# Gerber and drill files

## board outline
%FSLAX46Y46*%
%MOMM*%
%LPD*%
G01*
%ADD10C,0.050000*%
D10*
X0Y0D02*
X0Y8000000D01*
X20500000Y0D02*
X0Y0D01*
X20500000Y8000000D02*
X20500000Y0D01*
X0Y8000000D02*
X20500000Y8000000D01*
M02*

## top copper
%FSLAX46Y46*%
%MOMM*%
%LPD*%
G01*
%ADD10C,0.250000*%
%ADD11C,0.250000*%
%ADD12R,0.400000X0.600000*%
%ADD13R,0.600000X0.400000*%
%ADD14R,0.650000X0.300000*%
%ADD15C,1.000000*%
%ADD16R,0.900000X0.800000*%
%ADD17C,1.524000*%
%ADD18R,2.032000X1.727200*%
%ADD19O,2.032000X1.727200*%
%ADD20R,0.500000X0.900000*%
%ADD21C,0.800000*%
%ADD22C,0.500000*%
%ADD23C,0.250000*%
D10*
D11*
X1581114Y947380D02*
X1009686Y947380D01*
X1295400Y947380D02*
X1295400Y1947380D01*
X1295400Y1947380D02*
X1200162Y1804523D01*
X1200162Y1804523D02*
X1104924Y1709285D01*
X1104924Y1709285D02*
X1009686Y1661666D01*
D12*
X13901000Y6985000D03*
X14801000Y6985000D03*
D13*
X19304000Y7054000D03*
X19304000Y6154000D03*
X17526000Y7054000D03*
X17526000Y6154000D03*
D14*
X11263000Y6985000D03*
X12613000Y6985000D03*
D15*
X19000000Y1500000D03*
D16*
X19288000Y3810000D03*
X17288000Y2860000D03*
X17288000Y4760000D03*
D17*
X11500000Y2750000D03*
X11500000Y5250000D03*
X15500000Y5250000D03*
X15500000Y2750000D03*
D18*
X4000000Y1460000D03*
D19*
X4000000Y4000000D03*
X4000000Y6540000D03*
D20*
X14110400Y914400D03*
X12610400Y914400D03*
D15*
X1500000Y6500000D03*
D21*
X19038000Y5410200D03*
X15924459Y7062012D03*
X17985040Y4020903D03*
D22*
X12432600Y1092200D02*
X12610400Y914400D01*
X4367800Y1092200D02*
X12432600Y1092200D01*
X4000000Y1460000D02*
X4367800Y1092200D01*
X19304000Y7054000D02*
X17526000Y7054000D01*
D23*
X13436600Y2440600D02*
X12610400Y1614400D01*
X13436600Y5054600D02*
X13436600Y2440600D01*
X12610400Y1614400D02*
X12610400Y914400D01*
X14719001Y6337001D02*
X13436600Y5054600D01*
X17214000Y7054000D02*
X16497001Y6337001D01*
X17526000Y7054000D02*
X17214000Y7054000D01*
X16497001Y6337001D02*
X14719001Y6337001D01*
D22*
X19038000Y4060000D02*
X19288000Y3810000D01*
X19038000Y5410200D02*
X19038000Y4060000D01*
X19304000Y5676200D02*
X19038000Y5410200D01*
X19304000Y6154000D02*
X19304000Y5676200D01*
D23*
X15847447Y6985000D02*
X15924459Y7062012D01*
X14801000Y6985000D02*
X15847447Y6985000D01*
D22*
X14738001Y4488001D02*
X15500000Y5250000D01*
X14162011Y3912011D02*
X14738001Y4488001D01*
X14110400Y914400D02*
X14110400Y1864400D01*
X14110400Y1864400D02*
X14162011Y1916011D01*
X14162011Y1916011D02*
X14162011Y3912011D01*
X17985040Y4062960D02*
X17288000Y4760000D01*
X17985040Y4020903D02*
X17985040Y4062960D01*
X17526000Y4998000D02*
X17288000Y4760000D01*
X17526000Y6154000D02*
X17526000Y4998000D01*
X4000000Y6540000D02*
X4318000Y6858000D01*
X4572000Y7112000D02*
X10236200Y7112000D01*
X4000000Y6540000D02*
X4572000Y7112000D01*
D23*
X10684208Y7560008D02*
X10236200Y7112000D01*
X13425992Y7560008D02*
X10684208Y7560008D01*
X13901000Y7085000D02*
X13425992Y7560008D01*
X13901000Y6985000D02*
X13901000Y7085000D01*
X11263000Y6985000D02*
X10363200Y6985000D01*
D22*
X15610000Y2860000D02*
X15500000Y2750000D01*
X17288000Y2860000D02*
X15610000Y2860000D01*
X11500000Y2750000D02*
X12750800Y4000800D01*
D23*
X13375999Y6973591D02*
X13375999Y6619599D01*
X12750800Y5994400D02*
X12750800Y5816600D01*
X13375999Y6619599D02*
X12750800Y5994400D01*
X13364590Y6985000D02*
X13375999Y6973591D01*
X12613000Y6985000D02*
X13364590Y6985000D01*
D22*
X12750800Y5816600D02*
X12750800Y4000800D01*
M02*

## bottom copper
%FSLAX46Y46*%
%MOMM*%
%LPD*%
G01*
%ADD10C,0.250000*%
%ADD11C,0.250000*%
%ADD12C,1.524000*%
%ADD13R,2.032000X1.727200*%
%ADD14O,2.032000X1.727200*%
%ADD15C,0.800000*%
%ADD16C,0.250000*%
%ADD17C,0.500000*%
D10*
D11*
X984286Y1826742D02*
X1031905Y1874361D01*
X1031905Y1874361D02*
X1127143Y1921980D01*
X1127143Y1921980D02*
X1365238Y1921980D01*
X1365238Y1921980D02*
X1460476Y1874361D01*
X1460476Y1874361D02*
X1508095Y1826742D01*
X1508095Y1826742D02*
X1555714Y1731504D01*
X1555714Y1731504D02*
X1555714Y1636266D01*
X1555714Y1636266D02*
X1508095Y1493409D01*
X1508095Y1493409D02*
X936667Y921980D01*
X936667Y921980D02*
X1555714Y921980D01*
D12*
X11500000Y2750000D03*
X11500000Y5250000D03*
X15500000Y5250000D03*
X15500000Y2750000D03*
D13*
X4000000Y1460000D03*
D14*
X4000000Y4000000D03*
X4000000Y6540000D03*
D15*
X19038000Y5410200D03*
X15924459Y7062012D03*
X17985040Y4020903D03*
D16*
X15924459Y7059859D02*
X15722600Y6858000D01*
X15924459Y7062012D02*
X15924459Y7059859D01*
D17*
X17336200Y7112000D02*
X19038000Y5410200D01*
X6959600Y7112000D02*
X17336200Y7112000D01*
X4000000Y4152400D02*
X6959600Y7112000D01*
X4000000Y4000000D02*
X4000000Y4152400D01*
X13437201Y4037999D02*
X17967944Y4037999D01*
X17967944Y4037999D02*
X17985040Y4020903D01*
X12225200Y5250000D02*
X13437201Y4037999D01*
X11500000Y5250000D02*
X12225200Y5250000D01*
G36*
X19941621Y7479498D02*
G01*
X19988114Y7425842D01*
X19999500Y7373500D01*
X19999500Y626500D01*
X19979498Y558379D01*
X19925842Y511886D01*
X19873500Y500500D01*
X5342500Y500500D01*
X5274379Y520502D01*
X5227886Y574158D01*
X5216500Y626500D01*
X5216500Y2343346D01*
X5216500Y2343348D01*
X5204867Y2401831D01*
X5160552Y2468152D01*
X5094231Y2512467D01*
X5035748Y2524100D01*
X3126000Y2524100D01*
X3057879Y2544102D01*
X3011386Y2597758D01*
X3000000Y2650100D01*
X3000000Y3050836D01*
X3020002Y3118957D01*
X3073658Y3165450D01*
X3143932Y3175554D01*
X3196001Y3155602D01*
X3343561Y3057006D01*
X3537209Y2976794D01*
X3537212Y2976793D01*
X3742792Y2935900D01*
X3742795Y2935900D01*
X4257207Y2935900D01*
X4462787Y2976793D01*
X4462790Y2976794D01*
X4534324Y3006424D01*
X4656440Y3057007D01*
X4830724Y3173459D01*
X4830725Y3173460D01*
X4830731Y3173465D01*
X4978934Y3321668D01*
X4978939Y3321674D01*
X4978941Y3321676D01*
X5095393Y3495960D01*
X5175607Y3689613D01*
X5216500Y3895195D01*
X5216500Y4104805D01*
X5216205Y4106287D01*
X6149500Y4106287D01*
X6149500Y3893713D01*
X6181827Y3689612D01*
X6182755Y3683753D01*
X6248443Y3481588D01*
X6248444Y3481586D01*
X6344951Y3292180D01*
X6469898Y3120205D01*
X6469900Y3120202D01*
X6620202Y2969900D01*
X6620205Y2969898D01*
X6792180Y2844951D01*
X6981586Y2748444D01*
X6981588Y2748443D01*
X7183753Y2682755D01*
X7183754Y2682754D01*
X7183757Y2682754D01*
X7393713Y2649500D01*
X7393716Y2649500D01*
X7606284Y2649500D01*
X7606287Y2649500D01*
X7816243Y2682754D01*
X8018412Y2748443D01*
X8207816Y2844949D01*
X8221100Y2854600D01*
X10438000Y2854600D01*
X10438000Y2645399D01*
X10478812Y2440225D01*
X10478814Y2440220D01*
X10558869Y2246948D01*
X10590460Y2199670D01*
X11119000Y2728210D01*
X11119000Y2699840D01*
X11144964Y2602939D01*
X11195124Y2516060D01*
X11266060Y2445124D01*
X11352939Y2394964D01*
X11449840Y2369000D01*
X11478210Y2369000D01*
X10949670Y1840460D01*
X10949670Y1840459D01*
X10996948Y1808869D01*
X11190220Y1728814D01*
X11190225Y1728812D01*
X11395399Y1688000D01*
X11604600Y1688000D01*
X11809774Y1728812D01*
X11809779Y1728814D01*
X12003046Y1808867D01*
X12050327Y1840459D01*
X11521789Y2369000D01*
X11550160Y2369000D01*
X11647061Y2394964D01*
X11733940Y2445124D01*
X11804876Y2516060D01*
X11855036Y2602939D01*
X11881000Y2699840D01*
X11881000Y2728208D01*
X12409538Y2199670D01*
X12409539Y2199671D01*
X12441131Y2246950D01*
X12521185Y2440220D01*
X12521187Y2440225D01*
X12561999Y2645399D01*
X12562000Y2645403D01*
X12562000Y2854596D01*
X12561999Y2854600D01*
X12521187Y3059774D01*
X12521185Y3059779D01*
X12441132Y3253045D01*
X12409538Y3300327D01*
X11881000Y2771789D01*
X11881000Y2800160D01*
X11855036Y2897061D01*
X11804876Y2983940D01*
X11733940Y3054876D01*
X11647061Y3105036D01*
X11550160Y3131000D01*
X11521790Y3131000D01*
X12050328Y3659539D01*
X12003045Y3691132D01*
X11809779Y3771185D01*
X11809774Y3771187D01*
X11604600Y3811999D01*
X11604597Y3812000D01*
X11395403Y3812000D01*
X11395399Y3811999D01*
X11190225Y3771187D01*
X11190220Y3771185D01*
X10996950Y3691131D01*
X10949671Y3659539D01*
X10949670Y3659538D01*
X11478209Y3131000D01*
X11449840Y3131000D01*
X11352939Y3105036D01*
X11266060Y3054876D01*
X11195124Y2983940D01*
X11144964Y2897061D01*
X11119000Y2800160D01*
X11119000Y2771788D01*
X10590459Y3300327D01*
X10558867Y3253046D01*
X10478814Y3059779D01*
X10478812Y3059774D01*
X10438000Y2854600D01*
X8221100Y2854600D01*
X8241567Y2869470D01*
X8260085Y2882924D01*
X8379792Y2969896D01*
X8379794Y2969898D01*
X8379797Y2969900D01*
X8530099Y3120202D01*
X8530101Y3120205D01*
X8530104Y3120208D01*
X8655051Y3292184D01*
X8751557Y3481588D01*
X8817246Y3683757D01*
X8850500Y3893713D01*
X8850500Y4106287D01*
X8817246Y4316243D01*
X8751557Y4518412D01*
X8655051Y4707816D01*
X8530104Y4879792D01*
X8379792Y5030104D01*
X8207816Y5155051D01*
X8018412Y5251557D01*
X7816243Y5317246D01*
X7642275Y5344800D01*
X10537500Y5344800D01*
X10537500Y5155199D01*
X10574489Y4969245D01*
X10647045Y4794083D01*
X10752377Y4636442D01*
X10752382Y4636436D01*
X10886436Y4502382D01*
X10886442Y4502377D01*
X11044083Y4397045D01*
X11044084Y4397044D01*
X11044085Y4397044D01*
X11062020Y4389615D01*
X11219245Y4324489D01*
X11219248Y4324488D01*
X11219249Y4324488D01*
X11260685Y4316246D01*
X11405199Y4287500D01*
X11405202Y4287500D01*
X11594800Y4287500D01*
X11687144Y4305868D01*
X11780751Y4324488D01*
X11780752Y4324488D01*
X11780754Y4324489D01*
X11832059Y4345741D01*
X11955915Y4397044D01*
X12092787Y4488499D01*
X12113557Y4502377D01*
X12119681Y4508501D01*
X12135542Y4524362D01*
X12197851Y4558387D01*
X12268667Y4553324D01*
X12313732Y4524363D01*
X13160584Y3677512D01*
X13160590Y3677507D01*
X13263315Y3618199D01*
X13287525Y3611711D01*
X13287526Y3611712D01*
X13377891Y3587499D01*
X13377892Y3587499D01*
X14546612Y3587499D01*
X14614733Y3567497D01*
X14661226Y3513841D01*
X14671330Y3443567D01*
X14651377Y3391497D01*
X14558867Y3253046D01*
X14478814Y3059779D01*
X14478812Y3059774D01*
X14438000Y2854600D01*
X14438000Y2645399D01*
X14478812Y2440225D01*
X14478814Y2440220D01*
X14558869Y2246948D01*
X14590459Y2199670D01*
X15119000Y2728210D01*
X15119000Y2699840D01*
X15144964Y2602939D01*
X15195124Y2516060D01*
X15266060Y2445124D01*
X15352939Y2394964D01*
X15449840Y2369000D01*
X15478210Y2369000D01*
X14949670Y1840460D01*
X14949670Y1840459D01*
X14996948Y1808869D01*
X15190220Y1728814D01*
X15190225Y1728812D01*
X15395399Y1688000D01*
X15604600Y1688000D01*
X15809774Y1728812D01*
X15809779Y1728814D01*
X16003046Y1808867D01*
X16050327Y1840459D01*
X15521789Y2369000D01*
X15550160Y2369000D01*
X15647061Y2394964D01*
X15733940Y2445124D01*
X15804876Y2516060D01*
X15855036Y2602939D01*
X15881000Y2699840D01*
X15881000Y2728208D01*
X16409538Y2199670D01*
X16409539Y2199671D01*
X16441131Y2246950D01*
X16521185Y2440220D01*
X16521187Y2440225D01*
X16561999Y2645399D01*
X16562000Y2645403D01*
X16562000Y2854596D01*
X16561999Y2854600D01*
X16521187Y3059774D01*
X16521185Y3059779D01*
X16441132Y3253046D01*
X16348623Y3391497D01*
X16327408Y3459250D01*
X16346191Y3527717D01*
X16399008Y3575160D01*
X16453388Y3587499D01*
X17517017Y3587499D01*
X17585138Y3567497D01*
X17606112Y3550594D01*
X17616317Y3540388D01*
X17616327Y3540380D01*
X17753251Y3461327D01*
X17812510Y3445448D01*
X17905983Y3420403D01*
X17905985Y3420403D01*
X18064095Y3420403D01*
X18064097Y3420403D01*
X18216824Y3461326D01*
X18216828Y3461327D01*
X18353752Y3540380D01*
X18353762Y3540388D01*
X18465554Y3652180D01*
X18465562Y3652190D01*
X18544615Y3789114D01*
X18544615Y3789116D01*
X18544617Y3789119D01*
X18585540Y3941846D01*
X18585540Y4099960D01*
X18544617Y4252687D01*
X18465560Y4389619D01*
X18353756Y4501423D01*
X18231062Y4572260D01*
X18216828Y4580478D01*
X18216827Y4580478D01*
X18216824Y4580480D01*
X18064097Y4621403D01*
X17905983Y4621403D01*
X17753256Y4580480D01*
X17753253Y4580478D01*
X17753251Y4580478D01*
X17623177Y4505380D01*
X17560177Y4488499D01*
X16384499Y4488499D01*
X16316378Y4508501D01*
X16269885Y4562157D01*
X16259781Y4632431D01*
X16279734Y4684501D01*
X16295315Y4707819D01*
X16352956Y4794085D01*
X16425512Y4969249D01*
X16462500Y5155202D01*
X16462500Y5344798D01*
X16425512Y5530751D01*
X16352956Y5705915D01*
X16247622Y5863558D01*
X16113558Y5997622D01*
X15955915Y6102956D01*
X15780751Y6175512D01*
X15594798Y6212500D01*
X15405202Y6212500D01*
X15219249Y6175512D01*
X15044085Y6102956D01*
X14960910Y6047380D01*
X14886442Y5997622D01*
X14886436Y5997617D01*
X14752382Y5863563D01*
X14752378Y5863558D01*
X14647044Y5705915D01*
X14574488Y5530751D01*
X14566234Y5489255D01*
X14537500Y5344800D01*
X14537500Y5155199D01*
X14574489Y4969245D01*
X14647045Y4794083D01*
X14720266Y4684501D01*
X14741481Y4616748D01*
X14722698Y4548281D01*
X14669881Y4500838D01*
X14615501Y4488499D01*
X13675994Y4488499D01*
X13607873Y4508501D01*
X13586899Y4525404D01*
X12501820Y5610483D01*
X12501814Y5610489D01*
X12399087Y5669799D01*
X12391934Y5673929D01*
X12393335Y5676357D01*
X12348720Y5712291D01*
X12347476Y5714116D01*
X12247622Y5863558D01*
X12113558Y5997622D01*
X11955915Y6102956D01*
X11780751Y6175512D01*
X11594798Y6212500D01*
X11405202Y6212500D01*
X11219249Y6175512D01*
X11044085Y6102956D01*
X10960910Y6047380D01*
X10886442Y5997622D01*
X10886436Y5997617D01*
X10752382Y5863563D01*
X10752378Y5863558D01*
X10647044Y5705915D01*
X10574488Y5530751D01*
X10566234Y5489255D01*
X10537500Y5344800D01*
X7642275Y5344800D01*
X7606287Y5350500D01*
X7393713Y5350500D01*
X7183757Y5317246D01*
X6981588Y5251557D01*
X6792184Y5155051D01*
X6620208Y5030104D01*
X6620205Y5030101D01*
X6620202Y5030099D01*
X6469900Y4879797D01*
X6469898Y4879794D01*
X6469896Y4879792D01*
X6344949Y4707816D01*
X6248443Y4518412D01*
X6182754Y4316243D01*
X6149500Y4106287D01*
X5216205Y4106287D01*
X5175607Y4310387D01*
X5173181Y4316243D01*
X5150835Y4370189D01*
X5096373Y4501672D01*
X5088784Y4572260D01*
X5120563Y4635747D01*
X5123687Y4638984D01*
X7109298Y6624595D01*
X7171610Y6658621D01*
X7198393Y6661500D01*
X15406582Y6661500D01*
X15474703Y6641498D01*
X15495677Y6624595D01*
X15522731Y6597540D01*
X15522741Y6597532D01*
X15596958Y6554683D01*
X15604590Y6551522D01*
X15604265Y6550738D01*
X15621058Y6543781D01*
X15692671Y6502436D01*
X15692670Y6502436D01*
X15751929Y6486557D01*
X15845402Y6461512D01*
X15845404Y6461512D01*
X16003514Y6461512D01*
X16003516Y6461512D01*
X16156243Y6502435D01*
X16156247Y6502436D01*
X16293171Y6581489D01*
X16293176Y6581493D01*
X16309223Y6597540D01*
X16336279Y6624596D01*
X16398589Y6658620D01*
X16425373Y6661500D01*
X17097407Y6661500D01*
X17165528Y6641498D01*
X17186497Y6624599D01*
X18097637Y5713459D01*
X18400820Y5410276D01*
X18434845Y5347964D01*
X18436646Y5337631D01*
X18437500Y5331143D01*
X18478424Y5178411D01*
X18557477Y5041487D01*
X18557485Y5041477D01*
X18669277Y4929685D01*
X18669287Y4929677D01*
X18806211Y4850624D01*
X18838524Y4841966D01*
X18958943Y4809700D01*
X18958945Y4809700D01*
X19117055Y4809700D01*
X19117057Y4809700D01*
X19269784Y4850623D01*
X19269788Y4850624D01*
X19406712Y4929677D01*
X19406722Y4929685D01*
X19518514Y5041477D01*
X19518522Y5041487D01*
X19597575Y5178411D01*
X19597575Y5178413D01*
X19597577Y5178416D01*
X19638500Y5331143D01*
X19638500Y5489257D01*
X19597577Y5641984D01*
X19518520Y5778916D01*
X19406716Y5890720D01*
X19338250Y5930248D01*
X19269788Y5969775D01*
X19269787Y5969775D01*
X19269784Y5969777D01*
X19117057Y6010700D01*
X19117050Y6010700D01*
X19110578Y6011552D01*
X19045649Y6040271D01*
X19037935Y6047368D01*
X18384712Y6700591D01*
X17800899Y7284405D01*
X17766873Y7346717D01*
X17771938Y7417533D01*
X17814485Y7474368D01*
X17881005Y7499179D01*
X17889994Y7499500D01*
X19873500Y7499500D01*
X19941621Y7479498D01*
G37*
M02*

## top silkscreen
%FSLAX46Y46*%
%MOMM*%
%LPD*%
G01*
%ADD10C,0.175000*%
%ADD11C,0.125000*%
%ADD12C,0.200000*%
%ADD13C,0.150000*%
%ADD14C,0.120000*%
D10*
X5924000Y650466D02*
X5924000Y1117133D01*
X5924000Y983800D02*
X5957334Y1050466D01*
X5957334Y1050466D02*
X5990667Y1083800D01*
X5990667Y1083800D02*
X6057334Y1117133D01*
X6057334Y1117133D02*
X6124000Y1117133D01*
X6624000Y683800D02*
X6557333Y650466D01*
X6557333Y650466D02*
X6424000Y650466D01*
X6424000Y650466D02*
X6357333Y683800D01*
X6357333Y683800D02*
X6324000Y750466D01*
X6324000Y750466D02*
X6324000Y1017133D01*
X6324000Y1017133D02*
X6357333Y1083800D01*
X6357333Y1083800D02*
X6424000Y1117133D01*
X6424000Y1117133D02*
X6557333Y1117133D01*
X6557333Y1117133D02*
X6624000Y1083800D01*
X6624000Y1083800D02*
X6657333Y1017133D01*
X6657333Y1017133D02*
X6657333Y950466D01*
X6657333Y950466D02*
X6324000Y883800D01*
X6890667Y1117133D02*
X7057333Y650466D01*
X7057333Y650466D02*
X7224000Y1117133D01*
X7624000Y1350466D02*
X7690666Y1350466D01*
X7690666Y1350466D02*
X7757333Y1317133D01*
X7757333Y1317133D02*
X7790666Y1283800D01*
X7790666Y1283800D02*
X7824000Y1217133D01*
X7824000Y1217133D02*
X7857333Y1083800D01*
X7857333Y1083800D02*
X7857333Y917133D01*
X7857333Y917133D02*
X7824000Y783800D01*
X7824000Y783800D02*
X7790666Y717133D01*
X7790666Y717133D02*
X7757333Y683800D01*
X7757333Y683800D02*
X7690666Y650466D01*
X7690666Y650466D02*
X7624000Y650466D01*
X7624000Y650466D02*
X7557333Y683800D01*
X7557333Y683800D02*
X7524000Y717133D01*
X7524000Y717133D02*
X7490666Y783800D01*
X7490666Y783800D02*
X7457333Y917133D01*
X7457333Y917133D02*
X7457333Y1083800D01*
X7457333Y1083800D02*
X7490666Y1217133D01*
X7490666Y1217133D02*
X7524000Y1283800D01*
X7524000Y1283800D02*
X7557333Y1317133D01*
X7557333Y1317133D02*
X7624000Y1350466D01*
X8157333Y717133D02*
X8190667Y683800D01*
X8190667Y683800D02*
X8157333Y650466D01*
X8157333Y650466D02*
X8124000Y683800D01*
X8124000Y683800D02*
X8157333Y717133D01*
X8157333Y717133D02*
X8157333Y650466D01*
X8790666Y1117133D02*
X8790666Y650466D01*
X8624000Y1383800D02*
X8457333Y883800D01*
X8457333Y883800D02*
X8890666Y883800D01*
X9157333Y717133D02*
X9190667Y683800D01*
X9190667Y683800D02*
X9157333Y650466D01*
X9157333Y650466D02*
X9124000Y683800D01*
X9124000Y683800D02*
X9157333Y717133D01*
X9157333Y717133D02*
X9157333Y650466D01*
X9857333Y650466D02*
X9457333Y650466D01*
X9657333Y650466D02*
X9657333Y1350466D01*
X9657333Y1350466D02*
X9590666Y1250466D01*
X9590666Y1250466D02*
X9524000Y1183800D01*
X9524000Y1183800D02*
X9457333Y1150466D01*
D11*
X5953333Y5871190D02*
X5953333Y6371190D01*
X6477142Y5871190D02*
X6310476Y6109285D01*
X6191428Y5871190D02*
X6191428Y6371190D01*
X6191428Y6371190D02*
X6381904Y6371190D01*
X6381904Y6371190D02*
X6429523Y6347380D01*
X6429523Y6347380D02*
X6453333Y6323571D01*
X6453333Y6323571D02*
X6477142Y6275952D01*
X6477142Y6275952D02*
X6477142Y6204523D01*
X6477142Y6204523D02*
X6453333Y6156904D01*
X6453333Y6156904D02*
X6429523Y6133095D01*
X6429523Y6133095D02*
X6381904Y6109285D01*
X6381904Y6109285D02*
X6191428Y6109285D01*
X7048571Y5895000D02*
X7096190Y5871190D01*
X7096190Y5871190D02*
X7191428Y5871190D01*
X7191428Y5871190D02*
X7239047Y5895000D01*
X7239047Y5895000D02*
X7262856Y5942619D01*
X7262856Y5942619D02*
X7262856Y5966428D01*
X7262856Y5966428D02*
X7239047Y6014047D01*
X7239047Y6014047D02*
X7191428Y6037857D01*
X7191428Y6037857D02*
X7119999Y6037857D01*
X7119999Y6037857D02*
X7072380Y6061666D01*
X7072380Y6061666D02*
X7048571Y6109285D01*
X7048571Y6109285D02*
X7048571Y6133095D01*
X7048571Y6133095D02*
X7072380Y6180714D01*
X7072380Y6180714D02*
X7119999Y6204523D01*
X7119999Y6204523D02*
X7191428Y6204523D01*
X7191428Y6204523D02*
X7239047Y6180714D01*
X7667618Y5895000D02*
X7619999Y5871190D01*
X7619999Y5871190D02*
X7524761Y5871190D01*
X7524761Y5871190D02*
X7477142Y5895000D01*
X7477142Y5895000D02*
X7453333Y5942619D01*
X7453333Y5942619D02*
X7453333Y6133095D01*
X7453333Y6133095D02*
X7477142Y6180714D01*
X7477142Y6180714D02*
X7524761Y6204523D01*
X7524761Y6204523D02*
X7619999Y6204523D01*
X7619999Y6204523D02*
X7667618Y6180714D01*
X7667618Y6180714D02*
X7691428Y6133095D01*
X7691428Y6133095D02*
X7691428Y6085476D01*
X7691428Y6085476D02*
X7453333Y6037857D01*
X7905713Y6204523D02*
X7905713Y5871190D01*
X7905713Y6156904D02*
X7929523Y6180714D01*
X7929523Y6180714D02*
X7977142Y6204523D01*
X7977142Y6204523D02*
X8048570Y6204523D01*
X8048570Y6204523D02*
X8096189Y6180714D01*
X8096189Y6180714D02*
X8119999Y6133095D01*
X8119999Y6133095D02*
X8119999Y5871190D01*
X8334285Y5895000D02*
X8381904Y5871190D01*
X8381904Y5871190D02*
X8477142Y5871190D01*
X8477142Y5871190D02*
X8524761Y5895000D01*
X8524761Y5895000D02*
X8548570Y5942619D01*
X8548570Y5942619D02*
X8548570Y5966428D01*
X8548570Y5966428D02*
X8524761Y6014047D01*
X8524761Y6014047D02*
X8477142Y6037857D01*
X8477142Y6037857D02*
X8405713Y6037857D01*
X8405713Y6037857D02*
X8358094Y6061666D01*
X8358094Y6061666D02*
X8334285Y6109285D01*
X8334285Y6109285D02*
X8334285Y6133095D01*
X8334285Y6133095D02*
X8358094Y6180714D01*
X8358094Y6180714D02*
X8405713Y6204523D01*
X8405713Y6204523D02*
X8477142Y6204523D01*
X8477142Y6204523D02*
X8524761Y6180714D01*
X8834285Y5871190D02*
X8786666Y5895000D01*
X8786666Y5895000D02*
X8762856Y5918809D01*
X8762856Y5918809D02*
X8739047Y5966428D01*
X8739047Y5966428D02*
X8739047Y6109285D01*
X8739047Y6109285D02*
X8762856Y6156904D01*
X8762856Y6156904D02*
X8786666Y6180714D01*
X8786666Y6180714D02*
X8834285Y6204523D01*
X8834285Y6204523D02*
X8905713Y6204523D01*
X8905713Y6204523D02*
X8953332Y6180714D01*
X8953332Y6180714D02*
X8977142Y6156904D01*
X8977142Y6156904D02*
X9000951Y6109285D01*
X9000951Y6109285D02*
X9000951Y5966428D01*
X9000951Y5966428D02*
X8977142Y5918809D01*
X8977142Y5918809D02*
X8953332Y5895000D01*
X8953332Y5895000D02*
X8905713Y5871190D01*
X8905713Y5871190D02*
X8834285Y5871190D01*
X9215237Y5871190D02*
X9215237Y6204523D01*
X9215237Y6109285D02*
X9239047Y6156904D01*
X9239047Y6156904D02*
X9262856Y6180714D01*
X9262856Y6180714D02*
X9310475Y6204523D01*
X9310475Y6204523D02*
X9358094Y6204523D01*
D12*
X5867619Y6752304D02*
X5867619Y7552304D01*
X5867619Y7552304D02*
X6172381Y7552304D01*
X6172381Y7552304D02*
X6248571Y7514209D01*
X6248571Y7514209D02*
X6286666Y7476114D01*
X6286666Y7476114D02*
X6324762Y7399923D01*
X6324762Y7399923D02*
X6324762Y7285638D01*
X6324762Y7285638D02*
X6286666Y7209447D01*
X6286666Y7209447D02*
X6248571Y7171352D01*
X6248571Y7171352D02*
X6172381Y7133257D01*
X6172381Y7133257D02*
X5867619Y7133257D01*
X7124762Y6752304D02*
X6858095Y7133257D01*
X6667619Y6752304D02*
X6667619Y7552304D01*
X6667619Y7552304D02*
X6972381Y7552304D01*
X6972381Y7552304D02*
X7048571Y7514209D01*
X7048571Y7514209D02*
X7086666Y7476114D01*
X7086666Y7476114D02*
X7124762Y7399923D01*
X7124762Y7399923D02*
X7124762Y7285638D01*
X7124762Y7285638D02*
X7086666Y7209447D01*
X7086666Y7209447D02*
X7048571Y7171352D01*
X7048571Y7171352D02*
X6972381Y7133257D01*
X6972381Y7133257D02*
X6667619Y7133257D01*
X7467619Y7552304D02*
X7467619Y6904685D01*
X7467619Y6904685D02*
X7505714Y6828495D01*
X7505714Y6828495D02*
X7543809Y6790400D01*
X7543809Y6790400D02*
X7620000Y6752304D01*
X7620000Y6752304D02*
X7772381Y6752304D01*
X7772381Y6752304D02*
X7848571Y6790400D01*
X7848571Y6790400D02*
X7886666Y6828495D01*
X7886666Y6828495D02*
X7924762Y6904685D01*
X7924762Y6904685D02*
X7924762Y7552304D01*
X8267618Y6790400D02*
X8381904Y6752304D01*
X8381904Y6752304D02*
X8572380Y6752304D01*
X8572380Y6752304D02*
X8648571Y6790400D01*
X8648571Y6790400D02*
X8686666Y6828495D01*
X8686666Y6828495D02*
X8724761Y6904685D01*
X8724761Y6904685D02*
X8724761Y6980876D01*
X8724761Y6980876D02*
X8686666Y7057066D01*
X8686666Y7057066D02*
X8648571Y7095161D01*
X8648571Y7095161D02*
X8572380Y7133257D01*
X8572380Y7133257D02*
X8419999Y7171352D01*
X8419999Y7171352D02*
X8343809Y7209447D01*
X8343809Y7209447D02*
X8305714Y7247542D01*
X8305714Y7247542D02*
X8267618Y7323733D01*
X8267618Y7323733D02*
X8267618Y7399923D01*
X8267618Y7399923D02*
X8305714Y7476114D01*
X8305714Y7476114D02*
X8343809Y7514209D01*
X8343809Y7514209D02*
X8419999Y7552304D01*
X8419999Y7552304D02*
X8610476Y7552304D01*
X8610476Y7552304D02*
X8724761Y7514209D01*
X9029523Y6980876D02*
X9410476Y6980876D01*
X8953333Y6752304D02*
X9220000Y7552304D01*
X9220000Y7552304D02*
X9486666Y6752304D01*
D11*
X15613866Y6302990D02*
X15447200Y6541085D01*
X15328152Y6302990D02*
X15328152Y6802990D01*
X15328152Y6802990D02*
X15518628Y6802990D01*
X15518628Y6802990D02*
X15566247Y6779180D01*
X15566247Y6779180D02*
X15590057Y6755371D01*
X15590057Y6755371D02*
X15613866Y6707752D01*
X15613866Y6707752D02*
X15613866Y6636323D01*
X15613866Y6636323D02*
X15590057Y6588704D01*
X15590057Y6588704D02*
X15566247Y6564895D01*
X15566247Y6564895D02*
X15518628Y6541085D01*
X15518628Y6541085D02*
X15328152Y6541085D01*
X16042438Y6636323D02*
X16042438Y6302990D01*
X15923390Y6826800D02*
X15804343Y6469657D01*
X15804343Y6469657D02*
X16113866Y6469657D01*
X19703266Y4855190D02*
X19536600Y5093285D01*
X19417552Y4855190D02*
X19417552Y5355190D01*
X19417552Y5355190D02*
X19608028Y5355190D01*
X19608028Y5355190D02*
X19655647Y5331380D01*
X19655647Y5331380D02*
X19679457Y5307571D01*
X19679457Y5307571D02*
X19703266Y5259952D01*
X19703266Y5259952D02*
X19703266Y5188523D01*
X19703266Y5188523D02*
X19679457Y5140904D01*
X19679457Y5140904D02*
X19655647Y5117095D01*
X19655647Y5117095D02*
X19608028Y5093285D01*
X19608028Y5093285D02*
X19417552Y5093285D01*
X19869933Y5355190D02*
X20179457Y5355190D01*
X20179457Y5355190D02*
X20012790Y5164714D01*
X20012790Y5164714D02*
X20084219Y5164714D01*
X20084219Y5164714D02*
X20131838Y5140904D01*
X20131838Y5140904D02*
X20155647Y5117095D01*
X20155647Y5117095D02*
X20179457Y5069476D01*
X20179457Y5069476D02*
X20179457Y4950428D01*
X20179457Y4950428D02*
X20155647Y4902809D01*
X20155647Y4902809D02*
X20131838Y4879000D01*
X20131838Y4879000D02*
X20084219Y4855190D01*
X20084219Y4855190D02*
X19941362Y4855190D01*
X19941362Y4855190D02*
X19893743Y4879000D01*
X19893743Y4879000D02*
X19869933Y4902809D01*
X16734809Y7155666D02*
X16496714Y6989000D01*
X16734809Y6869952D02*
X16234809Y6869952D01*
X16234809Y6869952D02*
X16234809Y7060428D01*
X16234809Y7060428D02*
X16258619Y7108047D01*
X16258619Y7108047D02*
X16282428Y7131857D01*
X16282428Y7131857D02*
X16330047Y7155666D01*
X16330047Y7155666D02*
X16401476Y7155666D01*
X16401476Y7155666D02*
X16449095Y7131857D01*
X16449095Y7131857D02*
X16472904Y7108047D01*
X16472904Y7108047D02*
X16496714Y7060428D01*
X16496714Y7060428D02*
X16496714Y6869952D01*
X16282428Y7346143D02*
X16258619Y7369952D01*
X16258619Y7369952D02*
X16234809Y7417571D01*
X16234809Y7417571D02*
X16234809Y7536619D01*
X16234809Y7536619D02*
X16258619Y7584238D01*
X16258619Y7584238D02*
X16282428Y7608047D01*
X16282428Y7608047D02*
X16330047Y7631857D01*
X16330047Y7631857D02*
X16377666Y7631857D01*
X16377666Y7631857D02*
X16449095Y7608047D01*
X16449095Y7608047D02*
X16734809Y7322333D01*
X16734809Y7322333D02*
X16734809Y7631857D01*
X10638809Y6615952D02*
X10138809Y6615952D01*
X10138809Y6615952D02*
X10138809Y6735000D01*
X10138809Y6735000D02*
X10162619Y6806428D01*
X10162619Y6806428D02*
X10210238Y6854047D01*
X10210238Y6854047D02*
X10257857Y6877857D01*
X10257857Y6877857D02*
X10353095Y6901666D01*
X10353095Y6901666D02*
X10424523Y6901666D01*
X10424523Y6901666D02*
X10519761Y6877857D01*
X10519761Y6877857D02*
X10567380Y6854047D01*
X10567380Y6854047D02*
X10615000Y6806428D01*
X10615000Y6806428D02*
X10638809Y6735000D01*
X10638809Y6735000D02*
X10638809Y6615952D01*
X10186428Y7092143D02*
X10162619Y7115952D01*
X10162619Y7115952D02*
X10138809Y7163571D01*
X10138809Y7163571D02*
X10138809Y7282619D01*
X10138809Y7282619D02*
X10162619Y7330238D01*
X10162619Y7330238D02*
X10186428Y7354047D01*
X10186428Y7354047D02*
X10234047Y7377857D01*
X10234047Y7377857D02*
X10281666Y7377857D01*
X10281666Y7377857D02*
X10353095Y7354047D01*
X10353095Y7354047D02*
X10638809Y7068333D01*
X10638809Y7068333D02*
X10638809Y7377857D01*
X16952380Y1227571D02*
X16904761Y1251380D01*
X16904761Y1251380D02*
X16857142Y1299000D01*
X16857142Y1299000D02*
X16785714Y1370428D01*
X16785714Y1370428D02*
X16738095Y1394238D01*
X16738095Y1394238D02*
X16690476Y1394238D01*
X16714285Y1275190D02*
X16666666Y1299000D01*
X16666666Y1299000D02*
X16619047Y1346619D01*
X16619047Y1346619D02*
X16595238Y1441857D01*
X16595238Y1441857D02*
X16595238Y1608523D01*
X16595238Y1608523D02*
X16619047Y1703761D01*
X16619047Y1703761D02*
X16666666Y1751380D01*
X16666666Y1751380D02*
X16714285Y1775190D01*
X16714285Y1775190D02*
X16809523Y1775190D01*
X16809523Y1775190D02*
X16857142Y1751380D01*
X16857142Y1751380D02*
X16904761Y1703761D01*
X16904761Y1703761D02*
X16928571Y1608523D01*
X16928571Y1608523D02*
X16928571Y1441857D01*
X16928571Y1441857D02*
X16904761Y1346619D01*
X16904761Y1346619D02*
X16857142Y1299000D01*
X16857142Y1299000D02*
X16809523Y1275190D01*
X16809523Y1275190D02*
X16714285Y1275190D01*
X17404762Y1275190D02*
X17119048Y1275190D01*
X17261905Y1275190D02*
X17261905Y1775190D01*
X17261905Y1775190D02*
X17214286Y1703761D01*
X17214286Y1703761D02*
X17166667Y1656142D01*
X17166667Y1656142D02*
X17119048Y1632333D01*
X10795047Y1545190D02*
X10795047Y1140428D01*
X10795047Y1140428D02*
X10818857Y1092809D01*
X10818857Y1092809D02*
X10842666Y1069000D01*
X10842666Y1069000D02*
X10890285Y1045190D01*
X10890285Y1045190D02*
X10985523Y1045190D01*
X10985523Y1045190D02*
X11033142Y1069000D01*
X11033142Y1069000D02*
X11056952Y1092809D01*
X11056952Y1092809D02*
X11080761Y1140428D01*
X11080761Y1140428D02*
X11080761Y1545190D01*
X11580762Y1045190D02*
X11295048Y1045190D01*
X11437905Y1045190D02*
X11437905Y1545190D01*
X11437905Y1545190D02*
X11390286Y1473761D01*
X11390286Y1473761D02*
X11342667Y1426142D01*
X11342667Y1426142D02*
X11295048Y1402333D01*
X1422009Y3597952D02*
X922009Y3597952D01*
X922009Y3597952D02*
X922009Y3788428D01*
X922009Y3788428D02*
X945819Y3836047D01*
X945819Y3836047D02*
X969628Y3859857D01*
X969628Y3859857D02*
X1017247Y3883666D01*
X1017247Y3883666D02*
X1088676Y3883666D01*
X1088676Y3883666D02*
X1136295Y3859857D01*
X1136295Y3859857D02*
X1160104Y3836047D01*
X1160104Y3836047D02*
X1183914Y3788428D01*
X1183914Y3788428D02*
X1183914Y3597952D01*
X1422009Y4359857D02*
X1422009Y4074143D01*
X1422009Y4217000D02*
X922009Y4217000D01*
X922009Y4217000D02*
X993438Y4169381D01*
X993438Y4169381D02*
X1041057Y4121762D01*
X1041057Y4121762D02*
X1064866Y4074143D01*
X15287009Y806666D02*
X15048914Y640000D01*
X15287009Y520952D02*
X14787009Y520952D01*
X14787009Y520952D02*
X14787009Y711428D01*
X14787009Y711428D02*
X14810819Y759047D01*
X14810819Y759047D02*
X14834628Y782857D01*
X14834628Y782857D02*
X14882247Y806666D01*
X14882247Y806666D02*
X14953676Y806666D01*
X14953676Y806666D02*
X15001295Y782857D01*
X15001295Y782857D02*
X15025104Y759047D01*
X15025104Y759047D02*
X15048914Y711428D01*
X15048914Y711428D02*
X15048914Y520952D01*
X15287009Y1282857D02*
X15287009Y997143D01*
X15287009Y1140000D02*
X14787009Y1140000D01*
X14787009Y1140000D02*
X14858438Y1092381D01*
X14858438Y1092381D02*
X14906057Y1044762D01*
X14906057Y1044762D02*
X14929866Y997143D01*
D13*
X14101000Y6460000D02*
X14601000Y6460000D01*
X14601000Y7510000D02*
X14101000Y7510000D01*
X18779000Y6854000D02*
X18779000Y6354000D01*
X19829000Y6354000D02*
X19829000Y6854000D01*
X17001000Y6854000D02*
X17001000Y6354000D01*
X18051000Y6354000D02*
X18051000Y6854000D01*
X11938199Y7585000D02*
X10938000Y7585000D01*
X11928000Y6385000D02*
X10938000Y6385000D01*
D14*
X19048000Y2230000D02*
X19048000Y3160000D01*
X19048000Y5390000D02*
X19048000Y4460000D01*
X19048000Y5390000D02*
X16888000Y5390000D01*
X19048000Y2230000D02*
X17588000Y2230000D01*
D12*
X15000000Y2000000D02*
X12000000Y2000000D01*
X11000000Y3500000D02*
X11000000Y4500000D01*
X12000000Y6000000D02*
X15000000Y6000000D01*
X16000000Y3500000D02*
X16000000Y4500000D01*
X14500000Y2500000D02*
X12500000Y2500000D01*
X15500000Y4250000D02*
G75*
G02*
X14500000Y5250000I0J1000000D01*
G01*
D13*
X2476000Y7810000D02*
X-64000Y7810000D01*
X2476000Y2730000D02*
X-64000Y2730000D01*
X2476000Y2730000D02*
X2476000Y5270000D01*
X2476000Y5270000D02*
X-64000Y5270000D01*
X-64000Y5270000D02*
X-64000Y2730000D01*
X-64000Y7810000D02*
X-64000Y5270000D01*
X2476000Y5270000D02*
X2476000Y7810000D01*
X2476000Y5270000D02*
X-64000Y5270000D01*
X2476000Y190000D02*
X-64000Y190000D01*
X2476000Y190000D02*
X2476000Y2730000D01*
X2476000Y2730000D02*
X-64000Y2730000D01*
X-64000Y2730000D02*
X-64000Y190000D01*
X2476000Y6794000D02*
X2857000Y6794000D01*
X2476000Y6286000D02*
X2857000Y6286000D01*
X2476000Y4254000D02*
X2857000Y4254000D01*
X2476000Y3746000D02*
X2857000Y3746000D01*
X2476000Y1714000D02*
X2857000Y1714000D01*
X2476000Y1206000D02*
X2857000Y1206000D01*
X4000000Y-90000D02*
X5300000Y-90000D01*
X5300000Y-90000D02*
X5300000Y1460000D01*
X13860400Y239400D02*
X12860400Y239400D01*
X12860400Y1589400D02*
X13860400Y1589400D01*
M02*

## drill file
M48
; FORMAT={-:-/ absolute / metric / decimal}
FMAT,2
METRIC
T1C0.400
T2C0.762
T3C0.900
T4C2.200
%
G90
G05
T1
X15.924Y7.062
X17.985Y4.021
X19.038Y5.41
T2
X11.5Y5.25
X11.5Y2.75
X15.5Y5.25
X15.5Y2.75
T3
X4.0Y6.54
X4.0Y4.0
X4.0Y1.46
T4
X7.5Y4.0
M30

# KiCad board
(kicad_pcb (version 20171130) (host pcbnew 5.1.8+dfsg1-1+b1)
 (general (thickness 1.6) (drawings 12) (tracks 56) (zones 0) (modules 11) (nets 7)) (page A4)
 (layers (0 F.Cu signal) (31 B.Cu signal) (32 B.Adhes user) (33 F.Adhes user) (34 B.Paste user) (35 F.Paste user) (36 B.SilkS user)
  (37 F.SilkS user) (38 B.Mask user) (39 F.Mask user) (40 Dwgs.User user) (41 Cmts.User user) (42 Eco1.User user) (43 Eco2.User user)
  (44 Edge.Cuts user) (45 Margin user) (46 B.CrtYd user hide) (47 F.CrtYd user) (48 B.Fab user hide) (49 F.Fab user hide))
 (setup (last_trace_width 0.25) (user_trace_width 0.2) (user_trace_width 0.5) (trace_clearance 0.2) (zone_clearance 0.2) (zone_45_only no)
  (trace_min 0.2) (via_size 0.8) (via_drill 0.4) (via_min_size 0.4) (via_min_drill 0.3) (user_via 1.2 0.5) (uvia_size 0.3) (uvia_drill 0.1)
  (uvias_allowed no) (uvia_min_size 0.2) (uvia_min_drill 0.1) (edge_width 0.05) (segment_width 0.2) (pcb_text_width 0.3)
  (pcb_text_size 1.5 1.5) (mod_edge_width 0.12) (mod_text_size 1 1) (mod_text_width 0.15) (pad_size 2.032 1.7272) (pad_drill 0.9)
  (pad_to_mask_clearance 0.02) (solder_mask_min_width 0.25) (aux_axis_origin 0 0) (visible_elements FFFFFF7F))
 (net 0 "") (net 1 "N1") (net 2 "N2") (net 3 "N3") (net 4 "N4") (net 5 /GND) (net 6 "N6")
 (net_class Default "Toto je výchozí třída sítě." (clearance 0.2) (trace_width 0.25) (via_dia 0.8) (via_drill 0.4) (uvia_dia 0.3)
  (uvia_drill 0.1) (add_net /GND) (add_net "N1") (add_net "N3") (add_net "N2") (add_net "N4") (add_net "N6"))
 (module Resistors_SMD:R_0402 (layer F.Cu) (at 14.351 -6.985)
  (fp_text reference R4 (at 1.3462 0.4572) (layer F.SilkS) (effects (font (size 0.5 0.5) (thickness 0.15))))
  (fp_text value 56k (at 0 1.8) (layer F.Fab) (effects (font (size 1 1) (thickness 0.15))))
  (fp_line (start -0.25 0.525) (end 0.25 0.525) (layer F.SilkS) (width 0.15))
  (fp_line (start 0.25 -0.525) (end -0.25 -0.525) (layer F.SilkS) (width 0.15))
  (pad 1 smd rect (at -0.45 0) (size 0.4 0.6) (layers F.Cu F.Paste F.Mask) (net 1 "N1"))
  (pad 2 smd rect (at 0.45 0) (size 0.4 0.6) (layers F.Cu F.Paste F.Mask) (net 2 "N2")))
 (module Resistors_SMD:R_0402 (layer F.Cu) (at 19.304 -6.604 90)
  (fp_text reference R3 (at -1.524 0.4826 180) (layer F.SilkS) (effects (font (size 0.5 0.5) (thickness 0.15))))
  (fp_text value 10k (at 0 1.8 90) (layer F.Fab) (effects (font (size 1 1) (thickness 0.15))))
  (fp_line (start 0.25 -0.525) (end -0.25 -0.525) (layer F.SilkS) (width 0.15))
  (fp_line (start -0.25 0.525) (end 0.25 0.525) (layer F.SilkS) (width 0.15))
  (pad 2 smd rect (at 0.45 0 90) (size 0.4 0.6) (layers F.Cu F.Paste F.Mask) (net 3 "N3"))
  (pad 1 smd rect (at -0.45 0 90) (size 0.4 0.6) (layers F.Cu F.Paste F.Mask) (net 2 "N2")))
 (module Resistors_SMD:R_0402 (layer F.Cu) (at 17.526 -6.604 270)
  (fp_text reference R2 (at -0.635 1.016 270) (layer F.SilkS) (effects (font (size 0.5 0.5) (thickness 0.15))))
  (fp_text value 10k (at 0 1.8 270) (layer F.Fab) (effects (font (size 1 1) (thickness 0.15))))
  (fp_line (start -0.25 0.525) (end 0.25 0.525) (layer F.SilkS) (width 0.15))
  (fp_line (start 0.25 -0.525) (end -0.25 -0.525) (layer F.SilkS) (width 0.15))
  (pad 1 smd rect (at -0.45 0 270) (size 0.4 0.6) (layers F.Cu F.Paste F.Mask) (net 3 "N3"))
  (pad 2 smd rect (at 0.45 0 270) (size 0.4 0.6) (layers F.Cu F.Paste F.Mask) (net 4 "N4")))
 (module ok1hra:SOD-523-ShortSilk (layer F.Cu) (at 11.938 -6.985)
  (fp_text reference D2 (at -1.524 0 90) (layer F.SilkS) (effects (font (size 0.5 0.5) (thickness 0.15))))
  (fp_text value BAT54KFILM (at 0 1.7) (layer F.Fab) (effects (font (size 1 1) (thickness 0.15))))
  (fp_line (start 0.000199 -0.6) (end -1 -0.6) (layer F.SilkS) (width 0.15))
  (fp_line (start -0.01 0.6) (end -1 0.6) (layer F.SilkS) (width 0.15))
  (pad 1 smd rect (at -0.675 0 180) (size 0.65 0.3) (layers F.Cu F.Paste F.Mask) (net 1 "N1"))
  (pad 2 smd rect (at 0.675 0 180) (size 0.65 0.3) (layers F.Cu F.Paste F.Mask) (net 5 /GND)))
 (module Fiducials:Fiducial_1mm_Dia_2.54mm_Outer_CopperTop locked (layer F.Cu) (at 19 -1.5)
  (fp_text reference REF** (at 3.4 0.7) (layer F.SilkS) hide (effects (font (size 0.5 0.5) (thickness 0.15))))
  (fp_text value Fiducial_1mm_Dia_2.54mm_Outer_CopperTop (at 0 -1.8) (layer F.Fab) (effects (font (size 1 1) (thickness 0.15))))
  (pad ~ smd circle (at 0 0) (size 1 1) (layers F.Cu F.Mask) (solder_mask_margin 0.77) (clearance 0.77)))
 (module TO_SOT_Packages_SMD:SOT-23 (layer F.Cu) (at 18.288 -3.81)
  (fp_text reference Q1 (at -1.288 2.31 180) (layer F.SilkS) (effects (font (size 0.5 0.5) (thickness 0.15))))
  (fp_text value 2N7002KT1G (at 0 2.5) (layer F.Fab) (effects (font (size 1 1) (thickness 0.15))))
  (fp_line (start 0.76 1.58) (end 0.76 0.65) (layer F.SilkS) (width 0.12))
  (fp_line (start 0.76 -1.58) (end 0.76 -0.65) (layer F.SilkS) (width 0.12))
  (fp_line (start 0.76 -1.58) (end -1.4 -1.58) (layer F.SilkS) (width 0.12))
  (fp_line (start 0.76 1.58) (end -0.7 1.58) (layer F.SilkS) (width 0.12))
  (pad 3 smd rect (at 1 0) (size 0.9 0.8) (layers F.Cu F.Paste F.Mask) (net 2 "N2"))
  (pad 2 smd rect (at -1 0.95) (size 0.9 0.8) (layers F.Cu F.Paste F.Mask) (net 5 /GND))
  (pad 1 smd rect (at -1 -0.95) (size 0.9 0.8) (layers F.Cu F.Paste F.Mask) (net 4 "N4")))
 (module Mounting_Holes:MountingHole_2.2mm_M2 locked (layer F.Cu) (at 7.5 -4)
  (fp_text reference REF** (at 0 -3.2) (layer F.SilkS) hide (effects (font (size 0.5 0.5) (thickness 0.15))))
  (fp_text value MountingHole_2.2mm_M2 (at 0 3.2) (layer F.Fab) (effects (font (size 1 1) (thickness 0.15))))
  (pad 1 np_thru_hole circle (at 0 0) (size 2.2 2.2) (drill 2.2) (layers *.Cu *.Mask)))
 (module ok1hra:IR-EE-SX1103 (layer F.Cu) (at 13.5 -4 180)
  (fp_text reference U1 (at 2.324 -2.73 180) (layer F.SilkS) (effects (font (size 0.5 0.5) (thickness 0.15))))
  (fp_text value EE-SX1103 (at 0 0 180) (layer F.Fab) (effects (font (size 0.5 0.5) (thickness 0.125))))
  (fp_line (start -1.5 -2) (end 1.5 -2) (layer F.SilkS) (width 0.2))
  (fp_line (start 2.5 -0.5) (end 2.5 0.5) (layer F.SilkS) (width 0.2))
  (fp_line (start 1.5 2) (end -1.5 2) (layer F.SilkS) (width 0.2))
  (fp_line (start -2.5 -0.5) (end -2.5 0.5) (layer F.SilkS) (width 0.2))
  (fp_line (start -1 -1.5) (end 1 -1.5) (layer F.SilkS) (width 0.2))
  (fp_arc (start -2 1.25) (end -1 1.25) (angle -90) (layer F.SilkS) (width 0.2))
  (pad 3 thru_hole circle (at 2 -1.25 180) (size 1.524 1.524) (drill 0.762) (layers *.Cu *.Mask) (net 5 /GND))
  (pad 4 thru_hole circle (at 2 1.25 180) (size 1.524 1.524) (drill 0.762) (layers *.Cu *.Mask) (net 4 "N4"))
  (pad 1 thru_hole circle (at -2 1.25 180) (size 1.524 1.524) (drill 0.762) (layers *.Cu *.Mask) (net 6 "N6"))
  (pad 2 thru_hole circle (at -2 -1.25 180) (size 1.524 1.524) (drill 0.762) (layers *.Cu *.Mask) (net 5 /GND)))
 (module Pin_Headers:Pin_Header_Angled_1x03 (layer F.Cu) (at 4 -1.46 180)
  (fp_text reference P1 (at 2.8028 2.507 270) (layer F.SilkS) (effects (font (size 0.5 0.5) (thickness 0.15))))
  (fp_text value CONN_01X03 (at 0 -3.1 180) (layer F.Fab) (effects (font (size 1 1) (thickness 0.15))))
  (fp_line (start 1.524 6.35) (end 4.064 6.35) (layer F.SilkS) (width 0.15))
  (fp_line (start 1.524 1.27) (end 4.064 1.27) (layer F.SilkS) (width 0.15))
  (fp_line (start 1.524 1.27) (end 1.524 3.81) (layer F.SilkS) (width 0.15))
  (fp_line (start 1.524 3.81) (end 4.064 3.81) (layer F.SilkS) (width 0.15))
  (fp_line (start 4.064 3.81) (end 4.064 1.27) (layer F.SilkS) (width 0.15))
  (fp_line (start 4.064 6.35) (end 4.064 3.81) (layer F.SilkS) (width 0.15))
  (fp_line (start 1.524 3.81) (end 1.524 6.35) (layer F.SilkS) (width 0.15))
  (fp_line (start 1.524 3.81) (end 4.064 3.81) (layer F.SilkS) (width 0.15))
  (fp_line (start 1.524 -1.27) (end 4.064 -1.27) (layer F.SilkS) (width 0.15))
  (fp_line (start 1.524 -1.27) (end 1.524 1.27) (layer F.SilkS) (width 0.15))
  (fp_line (start 1.524 1.27) (end 4.064 1.27) (layer F.SilkS) (width 0.15))
  (fp_line (start 4.064 1.27) (end 4.064 -1.27) (layer F.SilkS) (width 0.15))
  (fp_line (start 1.524 5.334) (end 1.143 5.334) (layer F.SilkS) (width 0.15))
  (fp_line (start 1.524 4.826) (end 1.143 4.826) (layer F.SilkS) (width 0.15))
  (fp_line (start 1.524 2.794) (end 1.143 2.794) (layer F.SilkS) (width 0.15))
  (fp_line (start 1.524 2.286) (end 1.143 2.286) (layer F.SilkS) (width 0.15))
  (fp_line (start 1.524 0.254) (end 1.143 0.254) (layer F.SilkS) (width 0.15))
  (fp_line (start 1.524 -0.254) (end 1.143 -0.254) (layer F.SilkS) (width 0.15))
  (fp_line (start 0 -1.55) (end -1.3 -1.55) (layer F.SilkS) (width 0.15))
  (fp_line (start -1.3 -1.55) (end -1.3 0) (layer F.SilkS) (width 0.15))
  (pad 1 thru_hole rect (at 0 0 180) (size 2.032 1.7272) (drill 0.9) (layers *.Cu *.Mask) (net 3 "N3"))
  (pad 2 thru_hole oval (at 0 2.54 180) (size 2.032 1.7272) (drill 0.9) (layers *.Cu *.Mask) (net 2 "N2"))
  (pad 3 thru_hole oval (at 0 5.08 180) (size 2.032 1.7272) (drill 0.9) (layers *.Cu *.Mask) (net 1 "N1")))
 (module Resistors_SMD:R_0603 (layer F.Cu) (at 13.3604 -0.9144 180)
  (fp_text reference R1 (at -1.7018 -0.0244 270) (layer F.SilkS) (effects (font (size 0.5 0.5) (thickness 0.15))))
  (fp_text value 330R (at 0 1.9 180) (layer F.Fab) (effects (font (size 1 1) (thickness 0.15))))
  (fp_line (start -0.5 -0.675) (end 0.5 -0.675) (layer F.SilkS) (width 0.15))
  (fp_line (start 0.5 0.675) (end -0.5 0.675) (layer F.SilkS) (width 0.15))
  (pad 1 smd rect (at -0.75 0 180) (size 0.5 0.9) (layers F.Cu F.Paste F.Mask) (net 6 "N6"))
  (pad 2 smd rect (at 0.75 0 180) (size 0.5 0.9) (layers F.Cu F.Paste F.Mask) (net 3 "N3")))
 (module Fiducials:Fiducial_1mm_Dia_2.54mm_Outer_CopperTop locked (layer F.Cu) (at 1.5 -6.5)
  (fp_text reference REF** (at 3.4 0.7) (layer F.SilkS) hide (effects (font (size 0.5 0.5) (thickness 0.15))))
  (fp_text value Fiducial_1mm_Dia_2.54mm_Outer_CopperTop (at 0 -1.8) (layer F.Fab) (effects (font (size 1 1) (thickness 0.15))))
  (pad ~ smd circle (at 0 0) (size 1 1) (layers F.Cu F.Mask) (solder_mask_margin 0.77) (clearance 0.77)))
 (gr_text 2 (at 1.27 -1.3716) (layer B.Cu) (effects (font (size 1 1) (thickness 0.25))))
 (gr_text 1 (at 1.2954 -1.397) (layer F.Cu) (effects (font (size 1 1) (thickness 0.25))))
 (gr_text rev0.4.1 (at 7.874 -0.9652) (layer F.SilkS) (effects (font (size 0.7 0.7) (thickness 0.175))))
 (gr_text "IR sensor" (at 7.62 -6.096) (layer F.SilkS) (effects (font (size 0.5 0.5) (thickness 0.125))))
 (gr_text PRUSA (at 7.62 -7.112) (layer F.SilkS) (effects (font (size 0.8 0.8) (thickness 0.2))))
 (gr_line (start 0 0) (end 0 -8) (layer Edge.Cuts) (width 0.05))
 (gr_line (start 20.5 0) (end 0 0) (layer Edge.Cuts) (width 0.05))
 (gr_line (start 20.5 -8) (end 20.5 0) (layer Edge.Cuts) (width 0.05))
 (gr_line (start 0 -8) (end 20.5 -8) (layer Edge.Cuts) (width 0.05))
 (segment (start 12.4326 -1.0922) (end 12.6104 -0.9144) (width 0.5) (layer F.Cu) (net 3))
 (segment (start 4.3678 -1.0922) (end 12.4326 -1.0922) (width 0.5) (layer F.Cu) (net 3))
 (segment (start 4 -1.46) (end 4.3678 -1.0922) (width 0.5) (layer F.Cu) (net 3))
 (segment (start 19.304 -7.054) (end 17.526 -7.054) (width 0.5) (layer F.Cu) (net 3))
 (segment (start 13.4366 -2.4406) (end 12.6104 -1.6144) (width 0.25) (layer F.Cu) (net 3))
 (segment (start 13.4366 -5.0546) (end 13.4366 -2.4406) (width 0.25) (layer F.Cu) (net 3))
 (segment (start 12.6104 -1.6144) (end 12.6104 -0.9144) (width 0.25) (layer F.Cu) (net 3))
 (segment (start 14.719001 -6.337001) (end 13.4366 -5.0546) (width 0.25) (layer F.Cu) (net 3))
 (segment (start 17.214 -7.054) (end 16.497001 -6.337001) (width 0.25) (layer F.Cu) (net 3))
 (segment (start 17.526 -7.054) (end 17.214 -7.054) (width 0.25) (layer F.Cu) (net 3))
 (segment (start 16.497001 -6.337001) (end 14.719001 -6.337001) (width 0.25) (layer F.Cu) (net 3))
 (segment (start 19.038 -4.06) (end 19.288 -3.81) (width 0.5) (layer F.Cu) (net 2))
 (segment (start 19.038 -5.4102) (end 19.038 -4.06) (width 0.5) (layer F.Cu) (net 2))
 (via (at 19.038 -5.4102) (size 0.8) (drill 0.4) (layers F.Cu B.Cu) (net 2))
 (segment (start 19.304 -5.6762) (end 19.038 -5.4102) (width 0.5) (layer F.Cu) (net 2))
 (segment (start 19.304 -6.154) (end 19.304 -5.6762) (width 0.5) (layer F.Cu) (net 2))
 (via (at 15.924459 -7.062012) (size 0.8) (drill 0.4) (layers F.Cu B.Cu) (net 2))
 (segment (start 15.847447 -6.985) (end 15.924459 -7.062012) (width 0.25) (layer F.Cu) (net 2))
 (segment (start 14.801 -6.985) (end 15.847447 -6.985) (width 0.25) (layer F.Cu) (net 2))
 (segment (start 15.924459 -7.059859) (end 15.7226 -6.858) (width 0.25) (layer B.Cu) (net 2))
 (segment (start 15.924459 -7.062012) (end 15.924459 -7.059859) (width 0.25) (layer B.Cu) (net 2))
 (segment (start 17.3362 -7.112) (end 19.038 -5.4102) (width 0.5) (layer B.Cu) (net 2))
 (segment (start 6.9596 -7.112) (end 17.3362 -7.112) (width 0.5) (layer B.Cu) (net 2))
 (segment (start 4 -4.1524) (end 6.9596 -7.112) (width 0.5) (layer B.Cu) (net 2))
 (segment (start 4 -4) (end 4 -4.1524) (width 0.5) (layer B.Cu) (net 2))
 (segment (start 14.738001 -4.488001) (end 15.5 -5.25) (width 0.5) (layer F.Cu) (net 6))
 (segment (start 14.162011 -3.912011) (end 14.738001 -4.488001) (width 0.5) (layer F.Cu) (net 6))
 (segment (start 14.1104 -0.9144) (end 14.1104 -1.8644) (width 0.5) (layer F.Cu) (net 6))
 (segment (start 14.1104 -1.8644) (end 14.162011 -1.916011) (width 0.5) (layer F.Cu) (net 6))
 (segment (start 14.162011 -1.916011) (end 14.162011 -3.912011) (width 0.5) (layer F.Cu) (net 6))
 (via (at 17.98504 -4.020903) (size 0.8) (drill 0.4) (layers F.Cu B.Cu) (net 4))
 (segment (start 17.98504 -4.06296) (end 17.288 -4.76) (width 0.5) (layer F.Cu) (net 4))
 (segment (start 17.98504 -4.020903) (end 17.98504 -4.06296) (width 0.5) (layer F.Cu) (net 4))
 (segment (start 17.526 -4.998) (end 17.288 -4.76) (width 0.5) (layer F.Cu) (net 4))
 (segment (start 17.526 -6.154) (end 17.526 -4.998) (width 0.5) (layer F.Cu) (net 4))
 (segment (start 13.437201 -4.037999) (end 17.967944 -4.037999) (width 0.5) (layer B.Cu) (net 4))
 (segment (start 17.967944 -4.037999) (end 17.98504 -4.020903) (width 0.5) (layer B.Cu) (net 4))
 (segment (start 12.2252 -5.25) (end 13.437201 -4.037999) (width 0.5) (layer B.Cu) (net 4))
 (segment (start 11.5 -5.25) (end 12.2252 -5.25) (width 0.5) (layer B.Cu) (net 4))
 (segment (start 4 -6.54) (end 4.318 -6.858) (width 0.5) (layer F.Cu) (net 1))
 (segment (start 4.572 -7.112) (end 10.2362 -7.112) (width 0.5) (layer F.Cu) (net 1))
 (segment (start 4 -6.54) (end 4.572 -7.112) (width 0.5) (layer F.Cu) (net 1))
 (segment (start 10.684208 -7.560008) (end 10.2362 -7.112) (width 0.25) (layer F.Cu) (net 1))
 (segment (start 13.425992 -7.560008) (end 10.684208 -7.560008) (width 0.25) (layer F.Cu) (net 1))
 (segment (start 13.901 -7.085) (end 13.425992 -7.560008) (width 0.25) (layer F.Cu) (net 1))
 (segment (start 13.901 -6.985) (end 13.901 -7.085) (width 0.25) (layer F.Cu) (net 1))
 (segment (start 11.263 -6.985) (end 10.3632 -6.985) (width 0.25) (layer F.Cu) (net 1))
 (segment (start 15.61 -2.86) (end 15.5 -2.75) (width 0.5) (layer F.Cu) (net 5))
 (segment (start 17.288 -2.86) (end 15.61 -2.86) (width 0.5) (layer F.Cu) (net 5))
 (segment (start 11.5 -2.75) (end 12.7508 -4.0008) (width 0.5) (layer F.Cu) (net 5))
 (segment (start 13.375999 -6.973591) (end 13.375999 -6.619599) (width 0.25) (layer F.Cu) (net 5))
 (segment (start 12.7508 -5.9944) (end 12.7508 -5.8166) (width 0.25) (layer F.Cu) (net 5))
 (segment (start 13.375999 -6.619599) (end 12.7508 -5.9944) (width 0.25) (layer F.Cu) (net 5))
 (segment (start 13.36459 -6.985) (end 13.375999 -6.973591) (width 0.25) (layer F.Cu) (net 5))
 (segment (start 12.613 -6.985) (end 13.36459 -6.985) (width 0.25) (layer F.Cu) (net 5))
 (segment (start 12.7508 -5.8166) (end 12.7508 -4.0008) (width 0.5) (layer F.Cu) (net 5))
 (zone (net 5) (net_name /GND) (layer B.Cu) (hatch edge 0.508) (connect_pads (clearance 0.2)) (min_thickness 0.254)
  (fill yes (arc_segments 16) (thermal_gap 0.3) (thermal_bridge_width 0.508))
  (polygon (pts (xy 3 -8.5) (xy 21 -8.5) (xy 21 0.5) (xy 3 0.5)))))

